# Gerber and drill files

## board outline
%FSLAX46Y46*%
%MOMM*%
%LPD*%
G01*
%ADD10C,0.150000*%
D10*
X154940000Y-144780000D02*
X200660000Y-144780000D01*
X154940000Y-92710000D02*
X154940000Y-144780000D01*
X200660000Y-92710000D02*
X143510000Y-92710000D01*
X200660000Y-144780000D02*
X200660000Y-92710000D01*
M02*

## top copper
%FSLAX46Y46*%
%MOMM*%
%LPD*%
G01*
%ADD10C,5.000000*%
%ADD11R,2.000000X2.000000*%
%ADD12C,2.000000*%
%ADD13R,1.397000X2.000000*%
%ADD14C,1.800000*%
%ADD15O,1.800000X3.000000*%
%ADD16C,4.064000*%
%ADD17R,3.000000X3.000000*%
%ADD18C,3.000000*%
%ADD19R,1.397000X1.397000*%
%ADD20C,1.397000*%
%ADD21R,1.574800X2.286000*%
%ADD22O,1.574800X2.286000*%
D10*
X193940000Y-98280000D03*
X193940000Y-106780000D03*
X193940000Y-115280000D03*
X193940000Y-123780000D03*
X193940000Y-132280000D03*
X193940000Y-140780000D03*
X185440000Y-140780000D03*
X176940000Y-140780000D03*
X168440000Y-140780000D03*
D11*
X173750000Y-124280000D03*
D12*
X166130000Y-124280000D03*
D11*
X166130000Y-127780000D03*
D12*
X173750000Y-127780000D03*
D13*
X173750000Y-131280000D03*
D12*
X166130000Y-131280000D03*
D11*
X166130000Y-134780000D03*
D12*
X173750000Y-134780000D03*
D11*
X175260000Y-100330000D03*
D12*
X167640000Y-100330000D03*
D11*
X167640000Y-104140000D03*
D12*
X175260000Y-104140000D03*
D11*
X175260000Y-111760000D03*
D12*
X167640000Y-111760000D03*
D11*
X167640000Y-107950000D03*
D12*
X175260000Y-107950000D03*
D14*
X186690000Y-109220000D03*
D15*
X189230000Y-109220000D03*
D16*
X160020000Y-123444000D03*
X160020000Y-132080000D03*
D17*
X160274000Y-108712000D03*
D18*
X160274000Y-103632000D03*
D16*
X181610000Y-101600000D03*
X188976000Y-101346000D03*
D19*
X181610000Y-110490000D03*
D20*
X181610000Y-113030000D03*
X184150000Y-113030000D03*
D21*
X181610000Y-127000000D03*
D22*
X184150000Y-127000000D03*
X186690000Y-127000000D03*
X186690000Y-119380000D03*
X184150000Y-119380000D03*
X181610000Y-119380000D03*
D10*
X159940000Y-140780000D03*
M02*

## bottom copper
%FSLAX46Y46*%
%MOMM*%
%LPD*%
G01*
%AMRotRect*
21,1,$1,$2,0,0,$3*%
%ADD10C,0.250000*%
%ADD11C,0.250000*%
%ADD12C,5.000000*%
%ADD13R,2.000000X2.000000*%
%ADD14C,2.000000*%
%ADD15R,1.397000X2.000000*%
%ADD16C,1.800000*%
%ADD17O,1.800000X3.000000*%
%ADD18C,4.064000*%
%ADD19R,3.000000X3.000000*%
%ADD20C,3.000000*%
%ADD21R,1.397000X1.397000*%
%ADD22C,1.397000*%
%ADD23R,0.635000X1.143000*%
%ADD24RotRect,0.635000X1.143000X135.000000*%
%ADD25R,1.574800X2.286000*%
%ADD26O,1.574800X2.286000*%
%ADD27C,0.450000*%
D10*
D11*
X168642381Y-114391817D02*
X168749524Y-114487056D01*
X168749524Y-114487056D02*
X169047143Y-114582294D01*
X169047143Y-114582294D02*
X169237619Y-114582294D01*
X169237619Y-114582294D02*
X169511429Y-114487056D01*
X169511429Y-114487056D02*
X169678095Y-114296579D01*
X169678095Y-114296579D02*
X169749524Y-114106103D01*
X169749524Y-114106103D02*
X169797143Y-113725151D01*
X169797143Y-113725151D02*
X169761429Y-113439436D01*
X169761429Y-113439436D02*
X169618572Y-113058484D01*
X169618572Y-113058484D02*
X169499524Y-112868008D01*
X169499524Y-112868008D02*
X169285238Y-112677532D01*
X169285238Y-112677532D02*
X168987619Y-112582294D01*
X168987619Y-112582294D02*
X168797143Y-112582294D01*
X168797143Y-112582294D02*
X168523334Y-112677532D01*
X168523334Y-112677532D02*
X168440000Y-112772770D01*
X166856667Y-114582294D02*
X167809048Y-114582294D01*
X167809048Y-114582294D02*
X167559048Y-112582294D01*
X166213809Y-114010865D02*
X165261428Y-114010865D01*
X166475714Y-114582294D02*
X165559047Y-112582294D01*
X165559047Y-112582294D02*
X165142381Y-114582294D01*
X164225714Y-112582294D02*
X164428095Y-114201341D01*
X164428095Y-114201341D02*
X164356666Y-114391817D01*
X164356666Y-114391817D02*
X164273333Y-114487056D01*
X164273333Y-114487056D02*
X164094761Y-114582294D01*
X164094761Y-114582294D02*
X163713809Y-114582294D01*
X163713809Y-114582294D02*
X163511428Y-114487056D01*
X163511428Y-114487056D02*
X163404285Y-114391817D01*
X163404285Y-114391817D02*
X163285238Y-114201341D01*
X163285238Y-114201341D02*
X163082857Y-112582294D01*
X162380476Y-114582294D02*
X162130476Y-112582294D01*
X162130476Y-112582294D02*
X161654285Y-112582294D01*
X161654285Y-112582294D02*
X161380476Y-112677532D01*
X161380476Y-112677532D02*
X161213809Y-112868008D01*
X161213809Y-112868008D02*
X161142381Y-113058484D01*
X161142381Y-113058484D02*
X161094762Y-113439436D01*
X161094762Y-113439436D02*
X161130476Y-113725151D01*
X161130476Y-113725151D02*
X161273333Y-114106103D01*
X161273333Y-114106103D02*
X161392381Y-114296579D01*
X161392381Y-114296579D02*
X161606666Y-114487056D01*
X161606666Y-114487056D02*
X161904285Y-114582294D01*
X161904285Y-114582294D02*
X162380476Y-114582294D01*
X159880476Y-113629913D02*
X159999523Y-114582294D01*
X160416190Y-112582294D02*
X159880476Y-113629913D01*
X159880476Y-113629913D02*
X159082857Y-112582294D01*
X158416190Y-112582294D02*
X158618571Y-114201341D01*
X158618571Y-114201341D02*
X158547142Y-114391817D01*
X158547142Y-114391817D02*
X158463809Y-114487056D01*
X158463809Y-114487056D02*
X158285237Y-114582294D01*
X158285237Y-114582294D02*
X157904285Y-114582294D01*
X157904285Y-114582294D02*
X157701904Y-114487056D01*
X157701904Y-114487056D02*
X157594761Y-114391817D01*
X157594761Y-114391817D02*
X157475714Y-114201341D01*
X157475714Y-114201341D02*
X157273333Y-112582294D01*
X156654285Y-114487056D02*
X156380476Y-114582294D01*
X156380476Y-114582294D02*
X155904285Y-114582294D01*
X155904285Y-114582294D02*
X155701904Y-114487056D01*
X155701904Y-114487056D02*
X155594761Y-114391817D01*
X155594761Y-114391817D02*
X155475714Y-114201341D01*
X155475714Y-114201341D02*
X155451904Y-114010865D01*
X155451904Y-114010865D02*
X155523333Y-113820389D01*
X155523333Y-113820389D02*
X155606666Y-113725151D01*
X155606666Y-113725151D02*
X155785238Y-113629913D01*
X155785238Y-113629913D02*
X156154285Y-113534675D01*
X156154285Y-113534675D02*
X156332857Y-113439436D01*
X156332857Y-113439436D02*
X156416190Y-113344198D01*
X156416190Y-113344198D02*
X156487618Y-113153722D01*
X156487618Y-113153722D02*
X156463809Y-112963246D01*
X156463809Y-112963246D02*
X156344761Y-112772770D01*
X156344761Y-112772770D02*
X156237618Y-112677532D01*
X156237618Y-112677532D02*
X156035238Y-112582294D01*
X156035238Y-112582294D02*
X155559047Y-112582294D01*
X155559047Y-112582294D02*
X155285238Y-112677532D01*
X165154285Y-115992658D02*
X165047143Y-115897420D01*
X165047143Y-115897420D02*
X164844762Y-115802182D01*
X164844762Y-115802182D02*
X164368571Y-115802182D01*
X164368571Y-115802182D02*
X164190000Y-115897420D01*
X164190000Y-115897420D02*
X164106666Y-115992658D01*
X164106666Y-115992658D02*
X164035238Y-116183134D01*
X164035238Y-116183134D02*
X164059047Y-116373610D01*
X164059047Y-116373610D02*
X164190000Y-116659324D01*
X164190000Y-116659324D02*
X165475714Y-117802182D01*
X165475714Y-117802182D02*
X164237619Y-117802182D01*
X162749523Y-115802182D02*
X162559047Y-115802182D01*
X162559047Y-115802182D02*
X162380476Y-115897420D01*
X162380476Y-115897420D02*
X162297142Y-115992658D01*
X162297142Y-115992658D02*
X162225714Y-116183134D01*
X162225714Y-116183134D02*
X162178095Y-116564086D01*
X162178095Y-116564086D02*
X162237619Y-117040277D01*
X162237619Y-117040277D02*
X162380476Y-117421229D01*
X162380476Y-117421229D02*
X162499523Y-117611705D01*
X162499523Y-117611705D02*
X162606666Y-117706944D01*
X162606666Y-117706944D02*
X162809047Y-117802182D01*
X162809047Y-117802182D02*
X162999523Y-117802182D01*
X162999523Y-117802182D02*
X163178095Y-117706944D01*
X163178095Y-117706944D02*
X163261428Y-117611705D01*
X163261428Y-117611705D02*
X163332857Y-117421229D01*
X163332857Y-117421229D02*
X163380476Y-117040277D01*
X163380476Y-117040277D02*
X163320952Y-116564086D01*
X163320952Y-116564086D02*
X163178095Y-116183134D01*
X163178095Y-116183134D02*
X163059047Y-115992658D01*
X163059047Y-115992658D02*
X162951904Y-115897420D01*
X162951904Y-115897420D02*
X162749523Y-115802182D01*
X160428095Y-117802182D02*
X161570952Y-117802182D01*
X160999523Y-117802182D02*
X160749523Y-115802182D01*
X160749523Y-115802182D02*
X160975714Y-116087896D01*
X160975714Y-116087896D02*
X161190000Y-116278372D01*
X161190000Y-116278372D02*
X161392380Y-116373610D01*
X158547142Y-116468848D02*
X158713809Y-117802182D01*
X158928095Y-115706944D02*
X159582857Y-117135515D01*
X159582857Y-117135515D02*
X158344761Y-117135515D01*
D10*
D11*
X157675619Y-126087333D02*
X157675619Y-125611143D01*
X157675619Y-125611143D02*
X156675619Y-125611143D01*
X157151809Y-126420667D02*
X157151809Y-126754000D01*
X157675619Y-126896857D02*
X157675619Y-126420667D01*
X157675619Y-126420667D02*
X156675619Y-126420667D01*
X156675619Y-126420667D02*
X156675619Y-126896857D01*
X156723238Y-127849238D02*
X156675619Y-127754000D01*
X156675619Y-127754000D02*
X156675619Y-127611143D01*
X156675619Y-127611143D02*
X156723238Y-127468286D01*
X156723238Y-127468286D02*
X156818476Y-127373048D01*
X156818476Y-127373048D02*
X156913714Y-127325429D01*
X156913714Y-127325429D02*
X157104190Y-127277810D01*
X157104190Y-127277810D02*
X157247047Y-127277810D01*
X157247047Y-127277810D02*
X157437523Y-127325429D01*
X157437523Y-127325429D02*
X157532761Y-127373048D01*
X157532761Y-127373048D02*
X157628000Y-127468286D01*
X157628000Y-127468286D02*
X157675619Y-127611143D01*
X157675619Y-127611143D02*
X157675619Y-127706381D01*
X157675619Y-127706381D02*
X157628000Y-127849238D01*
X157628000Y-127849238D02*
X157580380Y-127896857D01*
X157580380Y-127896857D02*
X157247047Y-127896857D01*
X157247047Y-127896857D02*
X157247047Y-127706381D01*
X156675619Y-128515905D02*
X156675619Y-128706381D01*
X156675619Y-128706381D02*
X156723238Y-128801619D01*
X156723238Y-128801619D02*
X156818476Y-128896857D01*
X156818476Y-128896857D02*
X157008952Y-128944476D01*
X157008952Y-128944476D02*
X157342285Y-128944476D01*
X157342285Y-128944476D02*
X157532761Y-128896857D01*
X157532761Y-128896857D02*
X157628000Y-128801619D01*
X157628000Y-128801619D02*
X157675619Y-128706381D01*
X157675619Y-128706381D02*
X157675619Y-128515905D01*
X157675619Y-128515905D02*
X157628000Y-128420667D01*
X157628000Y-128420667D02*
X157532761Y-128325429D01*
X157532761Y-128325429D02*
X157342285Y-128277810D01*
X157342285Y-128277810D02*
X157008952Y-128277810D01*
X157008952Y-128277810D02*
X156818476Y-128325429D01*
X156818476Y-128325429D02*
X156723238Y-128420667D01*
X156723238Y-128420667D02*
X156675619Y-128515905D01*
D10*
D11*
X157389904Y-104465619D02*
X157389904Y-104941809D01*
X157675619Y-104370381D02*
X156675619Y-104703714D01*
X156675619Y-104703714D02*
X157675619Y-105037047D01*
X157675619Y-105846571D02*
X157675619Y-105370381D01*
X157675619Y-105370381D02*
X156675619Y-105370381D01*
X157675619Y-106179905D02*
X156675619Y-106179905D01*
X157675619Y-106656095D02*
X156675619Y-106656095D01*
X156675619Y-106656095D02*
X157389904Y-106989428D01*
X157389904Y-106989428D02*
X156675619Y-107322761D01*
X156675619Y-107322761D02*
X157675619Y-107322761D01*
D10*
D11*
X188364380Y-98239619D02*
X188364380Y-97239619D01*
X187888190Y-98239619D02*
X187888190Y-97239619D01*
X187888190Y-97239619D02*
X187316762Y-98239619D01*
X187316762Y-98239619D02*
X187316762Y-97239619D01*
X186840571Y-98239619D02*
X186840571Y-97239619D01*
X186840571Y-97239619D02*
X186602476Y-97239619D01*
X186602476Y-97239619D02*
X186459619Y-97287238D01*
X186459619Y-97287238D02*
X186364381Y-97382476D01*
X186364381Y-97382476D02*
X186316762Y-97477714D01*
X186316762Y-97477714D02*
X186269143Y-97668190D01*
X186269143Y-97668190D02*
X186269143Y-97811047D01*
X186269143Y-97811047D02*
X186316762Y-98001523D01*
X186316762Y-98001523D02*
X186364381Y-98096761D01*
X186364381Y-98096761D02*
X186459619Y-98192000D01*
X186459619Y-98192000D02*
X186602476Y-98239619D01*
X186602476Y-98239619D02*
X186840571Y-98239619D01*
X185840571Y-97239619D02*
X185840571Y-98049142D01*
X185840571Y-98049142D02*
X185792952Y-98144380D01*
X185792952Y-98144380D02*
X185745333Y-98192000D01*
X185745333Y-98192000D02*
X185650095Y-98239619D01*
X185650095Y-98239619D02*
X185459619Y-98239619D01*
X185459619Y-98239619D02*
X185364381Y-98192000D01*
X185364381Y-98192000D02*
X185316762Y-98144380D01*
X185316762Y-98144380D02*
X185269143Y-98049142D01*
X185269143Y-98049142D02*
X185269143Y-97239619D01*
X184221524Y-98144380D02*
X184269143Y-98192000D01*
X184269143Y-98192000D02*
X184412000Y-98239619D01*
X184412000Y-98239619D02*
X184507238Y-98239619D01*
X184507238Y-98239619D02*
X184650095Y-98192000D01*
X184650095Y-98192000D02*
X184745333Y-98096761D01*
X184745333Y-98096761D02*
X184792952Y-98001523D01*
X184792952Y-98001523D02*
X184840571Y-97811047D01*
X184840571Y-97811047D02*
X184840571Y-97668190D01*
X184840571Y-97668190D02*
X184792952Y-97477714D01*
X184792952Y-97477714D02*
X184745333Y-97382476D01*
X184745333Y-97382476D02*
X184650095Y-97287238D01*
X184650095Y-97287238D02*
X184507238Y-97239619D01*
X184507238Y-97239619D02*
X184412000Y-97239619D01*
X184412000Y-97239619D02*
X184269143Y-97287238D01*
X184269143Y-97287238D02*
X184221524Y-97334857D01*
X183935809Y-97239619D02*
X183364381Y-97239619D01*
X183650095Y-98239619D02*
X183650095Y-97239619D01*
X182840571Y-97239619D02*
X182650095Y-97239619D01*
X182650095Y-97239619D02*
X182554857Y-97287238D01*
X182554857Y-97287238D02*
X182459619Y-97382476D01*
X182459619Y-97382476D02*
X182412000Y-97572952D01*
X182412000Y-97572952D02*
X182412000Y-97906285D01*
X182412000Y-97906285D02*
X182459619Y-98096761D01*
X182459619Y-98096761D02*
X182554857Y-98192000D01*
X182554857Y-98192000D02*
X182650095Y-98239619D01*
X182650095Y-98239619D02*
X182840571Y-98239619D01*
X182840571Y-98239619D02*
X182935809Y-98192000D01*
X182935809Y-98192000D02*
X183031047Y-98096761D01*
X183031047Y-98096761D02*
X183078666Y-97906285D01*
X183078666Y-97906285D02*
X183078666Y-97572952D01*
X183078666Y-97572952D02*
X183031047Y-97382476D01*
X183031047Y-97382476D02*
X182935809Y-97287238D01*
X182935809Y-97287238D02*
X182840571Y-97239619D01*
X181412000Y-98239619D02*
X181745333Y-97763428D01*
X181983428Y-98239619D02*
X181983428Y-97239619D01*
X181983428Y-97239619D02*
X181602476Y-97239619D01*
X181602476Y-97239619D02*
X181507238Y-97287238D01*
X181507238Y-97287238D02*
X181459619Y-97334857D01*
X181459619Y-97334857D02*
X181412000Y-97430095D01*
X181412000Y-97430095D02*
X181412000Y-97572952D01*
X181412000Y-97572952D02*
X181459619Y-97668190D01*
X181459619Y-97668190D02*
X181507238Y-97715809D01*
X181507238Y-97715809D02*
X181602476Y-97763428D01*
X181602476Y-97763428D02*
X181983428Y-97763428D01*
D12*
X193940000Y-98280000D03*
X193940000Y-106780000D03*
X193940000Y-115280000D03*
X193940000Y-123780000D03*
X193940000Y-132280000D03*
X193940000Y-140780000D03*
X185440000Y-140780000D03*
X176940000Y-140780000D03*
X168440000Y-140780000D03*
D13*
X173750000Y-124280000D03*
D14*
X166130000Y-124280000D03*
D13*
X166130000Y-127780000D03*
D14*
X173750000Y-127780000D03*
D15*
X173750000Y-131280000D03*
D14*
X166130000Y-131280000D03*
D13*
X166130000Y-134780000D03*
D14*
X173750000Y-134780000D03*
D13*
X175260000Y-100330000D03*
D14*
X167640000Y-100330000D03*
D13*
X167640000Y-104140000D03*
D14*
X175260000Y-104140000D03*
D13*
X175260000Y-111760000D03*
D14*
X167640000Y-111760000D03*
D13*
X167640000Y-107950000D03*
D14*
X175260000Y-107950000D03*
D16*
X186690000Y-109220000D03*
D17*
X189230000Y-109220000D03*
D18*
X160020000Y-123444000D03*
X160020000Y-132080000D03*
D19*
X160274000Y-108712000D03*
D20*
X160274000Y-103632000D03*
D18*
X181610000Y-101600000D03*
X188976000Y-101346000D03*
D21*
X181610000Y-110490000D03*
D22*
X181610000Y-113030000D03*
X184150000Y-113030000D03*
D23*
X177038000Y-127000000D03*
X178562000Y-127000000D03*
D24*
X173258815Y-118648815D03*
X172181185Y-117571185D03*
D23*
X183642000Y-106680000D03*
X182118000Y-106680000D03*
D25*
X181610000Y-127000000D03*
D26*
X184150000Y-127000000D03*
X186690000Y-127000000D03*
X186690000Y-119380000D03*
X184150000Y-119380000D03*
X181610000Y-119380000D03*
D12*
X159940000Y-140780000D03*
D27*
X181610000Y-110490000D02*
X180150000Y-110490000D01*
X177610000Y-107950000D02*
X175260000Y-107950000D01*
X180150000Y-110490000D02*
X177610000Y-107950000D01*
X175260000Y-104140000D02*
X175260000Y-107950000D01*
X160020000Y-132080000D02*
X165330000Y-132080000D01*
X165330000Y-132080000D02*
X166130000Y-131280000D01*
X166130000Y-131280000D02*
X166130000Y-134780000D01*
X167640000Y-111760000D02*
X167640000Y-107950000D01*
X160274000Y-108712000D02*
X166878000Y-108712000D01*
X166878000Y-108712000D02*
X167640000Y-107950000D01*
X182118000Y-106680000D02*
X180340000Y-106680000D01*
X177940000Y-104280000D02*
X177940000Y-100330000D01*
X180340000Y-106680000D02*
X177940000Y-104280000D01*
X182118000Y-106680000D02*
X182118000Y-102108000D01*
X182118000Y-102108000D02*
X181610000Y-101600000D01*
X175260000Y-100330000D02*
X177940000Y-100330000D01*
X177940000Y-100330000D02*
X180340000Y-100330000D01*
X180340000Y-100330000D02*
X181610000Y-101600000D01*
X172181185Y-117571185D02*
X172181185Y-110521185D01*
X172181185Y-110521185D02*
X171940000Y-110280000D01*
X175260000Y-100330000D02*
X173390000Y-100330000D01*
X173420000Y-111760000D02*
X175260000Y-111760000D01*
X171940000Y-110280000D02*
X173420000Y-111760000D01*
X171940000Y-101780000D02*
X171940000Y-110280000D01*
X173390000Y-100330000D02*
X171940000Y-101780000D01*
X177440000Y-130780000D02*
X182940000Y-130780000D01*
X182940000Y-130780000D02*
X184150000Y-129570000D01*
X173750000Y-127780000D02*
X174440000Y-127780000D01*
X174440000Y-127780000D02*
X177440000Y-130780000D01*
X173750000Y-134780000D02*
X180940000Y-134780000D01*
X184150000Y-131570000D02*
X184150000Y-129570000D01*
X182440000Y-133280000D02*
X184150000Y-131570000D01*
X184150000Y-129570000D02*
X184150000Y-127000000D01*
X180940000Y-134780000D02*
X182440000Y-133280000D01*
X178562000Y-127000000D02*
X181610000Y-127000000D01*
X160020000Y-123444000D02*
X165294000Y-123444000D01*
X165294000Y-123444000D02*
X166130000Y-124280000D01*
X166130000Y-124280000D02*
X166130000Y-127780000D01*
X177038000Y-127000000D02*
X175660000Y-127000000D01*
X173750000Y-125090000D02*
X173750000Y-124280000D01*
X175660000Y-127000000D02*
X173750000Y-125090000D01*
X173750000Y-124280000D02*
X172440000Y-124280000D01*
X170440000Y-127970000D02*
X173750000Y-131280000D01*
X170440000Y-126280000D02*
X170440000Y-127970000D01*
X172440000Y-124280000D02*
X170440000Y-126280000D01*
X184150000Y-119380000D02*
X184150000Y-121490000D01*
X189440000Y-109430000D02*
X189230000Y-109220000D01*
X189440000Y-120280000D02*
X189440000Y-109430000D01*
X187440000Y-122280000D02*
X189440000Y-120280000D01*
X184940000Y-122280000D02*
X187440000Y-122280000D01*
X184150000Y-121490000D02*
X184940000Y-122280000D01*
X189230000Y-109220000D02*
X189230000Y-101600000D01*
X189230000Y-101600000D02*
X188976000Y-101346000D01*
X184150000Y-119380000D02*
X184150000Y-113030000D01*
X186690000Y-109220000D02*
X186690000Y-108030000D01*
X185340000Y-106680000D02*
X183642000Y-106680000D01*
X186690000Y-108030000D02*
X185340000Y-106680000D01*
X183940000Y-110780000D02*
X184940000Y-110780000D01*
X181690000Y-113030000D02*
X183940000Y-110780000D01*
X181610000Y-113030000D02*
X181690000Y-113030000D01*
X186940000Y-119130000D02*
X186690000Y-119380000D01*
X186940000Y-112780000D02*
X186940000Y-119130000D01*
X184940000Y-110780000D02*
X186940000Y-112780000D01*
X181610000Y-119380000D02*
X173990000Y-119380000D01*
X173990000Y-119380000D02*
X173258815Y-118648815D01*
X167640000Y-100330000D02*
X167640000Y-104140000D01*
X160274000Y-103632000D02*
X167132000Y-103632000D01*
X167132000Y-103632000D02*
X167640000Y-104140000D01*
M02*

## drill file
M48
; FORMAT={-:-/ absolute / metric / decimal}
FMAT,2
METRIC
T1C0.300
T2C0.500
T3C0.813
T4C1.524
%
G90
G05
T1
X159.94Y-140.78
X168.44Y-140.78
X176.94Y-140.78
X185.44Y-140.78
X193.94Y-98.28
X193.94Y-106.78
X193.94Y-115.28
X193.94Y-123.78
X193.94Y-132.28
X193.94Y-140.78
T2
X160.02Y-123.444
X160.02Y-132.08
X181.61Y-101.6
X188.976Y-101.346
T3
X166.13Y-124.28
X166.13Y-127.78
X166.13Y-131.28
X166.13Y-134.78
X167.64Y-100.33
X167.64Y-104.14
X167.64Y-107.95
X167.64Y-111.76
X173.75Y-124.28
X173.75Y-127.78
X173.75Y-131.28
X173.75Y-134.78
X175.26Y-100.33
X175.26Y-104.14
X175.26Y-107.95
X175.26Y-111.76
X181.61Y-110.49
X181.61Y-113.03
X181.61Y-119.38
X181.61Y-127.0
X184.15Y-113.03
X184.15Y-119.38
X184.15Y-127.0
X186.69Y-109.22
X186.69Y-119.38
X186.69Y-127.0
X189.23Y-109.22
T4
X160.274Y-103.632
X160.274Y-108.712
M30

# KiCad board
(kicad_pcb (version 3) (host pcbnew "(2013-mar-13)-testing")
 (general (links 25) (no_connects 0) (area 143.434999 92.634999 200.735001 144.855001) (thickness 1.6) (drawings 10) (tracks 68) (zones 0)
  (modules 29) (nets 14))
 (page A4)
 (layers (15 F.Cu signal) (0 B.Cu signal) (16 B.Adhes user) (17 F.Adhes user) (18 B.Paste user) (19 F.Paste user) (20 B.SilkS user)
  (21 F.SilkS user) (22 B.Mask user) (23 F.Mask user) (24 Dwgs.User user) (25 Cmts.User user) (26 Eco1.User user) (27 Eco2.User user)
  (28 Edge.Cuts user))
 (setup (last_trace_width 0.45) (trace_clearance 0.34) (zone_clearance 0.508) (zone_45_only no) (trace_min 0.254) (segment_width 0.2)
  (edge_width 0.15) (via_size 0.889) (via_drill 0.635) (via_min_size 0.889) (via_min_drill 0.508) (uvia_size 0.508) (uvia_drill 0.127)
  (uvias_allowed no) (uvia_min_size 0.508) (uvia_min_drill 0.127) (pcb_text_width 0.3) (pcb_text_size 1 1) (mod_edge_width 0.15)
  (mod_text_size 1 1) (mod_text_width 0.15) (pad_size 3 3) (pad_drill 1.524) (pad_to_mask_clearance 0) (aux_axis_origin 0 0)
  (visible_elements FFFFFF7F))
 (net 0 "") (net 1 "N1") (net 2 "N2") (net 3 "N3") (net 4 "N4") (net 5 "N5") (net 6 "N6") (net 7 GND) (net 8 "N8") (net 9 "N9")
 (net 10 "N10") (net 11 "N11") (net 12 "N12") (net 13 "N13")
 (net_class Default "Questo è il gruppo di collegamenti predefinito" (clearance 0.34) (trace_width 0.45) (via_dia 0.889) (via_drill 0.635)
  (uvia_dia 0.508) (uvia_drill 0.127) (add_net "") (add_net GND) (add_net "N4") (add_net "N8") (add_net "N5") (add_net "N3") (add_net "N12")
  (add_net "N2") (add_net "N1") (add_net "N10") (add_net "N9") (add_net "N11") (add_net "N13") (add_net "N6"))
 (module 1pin (layer F.Cu) (at 193.94 98.28)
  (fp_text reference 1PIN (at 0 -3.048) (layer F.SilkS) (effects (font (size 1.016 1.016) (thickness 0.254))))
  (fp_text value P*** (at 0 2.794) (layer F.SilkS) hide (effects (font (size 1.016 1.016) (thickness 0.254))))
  (pad 1 thru_hole circle (at 0 0) (size 5 5) (drill 0.3) (layers *.Cu *.Mask F.SilkS)))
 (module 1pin (layer F.Cu) (at 193.94 106.78)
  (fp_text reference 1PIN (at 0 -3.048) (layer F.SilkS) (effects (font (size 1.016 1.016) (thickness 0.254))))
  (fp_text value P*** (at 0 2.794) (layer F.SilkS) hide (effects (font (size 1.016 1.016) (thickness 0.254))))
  (pad 1 thru_hole circle (at 0 0) (size 5 5) (drill 0.3) (layers *.Cu *.Mask F.SilkS)))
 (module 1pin (layer F.Cu) (at 193.94 115.28)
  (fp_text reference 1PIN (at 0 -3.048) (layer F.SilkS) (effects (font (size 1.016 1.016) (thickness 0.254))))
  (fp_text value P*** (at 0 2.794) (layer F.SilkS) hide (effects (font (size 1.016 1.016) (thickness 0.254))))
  (pad 1 thru_hole circle (at 0 0) (size 5 5) (drill 0.3) (layers *.Cu *.Mask F.SilkS)))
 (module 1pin (layer F.Cu) (at 193.94 123.78)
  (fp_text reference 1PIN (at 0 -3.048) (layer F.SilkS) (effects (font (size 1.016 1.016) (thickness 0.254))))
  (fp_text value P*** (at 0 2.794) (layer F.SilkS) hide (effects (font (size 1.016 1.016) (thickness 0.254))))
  (pad 1 thru_hole circle (at 0 0) (size 5 5) (drill 0.3) (layers *.Cu *.Mask F.SilkS)))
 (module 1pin (layer F.Cu) (at 193.94 132.28)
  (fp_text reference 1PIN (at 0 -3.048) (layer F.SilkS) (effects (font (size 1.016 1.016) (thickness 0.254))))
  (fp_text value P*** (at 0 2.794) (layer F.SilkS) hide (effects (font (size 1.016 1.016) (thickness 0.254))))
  (pad 1 thru_hole circle (at 0 0) (size 5 5) (drill 0.3) (layers *.Cu *.Mask F.SilkS)))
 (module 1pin (layer F.Cu) (at 193.94 140.78)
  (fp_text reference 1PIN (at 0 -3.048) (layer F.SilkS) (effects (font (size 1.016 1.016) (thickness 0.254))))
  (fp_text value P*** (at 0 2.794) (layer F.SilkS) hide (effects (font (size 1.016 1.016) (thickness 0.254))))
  (pad 1 thru_hole circle (at 0 0) (size 5 5) (drill 0.3) (layers *.Cu *.Mask F.SilkS)))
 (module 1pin (layer F.Cu) (at 185.44 140.78)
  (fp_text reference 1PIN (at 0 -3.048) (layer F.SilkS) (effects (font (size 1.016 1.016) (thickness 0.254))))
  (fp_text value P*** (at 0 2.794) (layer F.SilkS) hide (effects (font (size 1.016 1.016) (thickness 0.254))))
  (pad 1 thru_hole circle (at 0 0) (size 5 5) (drill 0.3) (layers *.Cu *.Mask F.SilkS)))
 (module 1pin (layer F.Cu) (at 176.94 140.78)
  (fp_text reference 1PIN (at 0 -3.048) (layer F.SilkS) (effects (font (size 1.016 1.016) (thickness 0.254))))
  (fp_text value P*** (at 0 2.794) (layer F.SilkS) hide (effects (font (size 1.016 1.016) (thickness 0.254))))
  (pad 1 thru_hole circle (at 0 0) (size 5 5) (drill 0.3) (layers *.Cu *.Mask F.SilkS)))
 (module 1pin (layer F.Cu) (at 168.44 140.78)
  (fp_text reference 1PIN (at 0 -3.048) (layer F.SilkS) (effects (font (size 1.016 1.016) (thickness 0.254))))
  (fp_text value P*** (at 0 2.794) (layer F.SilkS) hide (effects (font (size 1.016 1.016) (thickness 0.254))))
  (pad 1 thru_hole circle (at 0 0) (size 5 5) (drill 0.3) (layers *.Cu *.Mask F.SilkS)))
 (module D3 (layer F.Cu) (at 169.94 124.28)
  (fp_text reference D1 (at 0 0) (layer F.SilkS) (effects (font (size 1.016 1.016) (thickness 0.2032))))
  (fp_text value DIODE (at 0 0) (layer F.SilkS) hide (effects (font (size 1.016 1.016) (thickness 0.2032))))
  (pad 2 thru_hole rect (at 3.81 0) (size 2 2) (drill 0.8128) (layers *.Cu *.Mask F.SilkS) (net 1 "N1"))
  (pad 1 thru_hole circle (at -3.81 0) (size 2 2) (drill 0.8128) (layers *.Cu *.Mask F.SilkS) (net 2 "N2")))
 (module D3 (layer F.Cu) (at 169.94 127.78 180)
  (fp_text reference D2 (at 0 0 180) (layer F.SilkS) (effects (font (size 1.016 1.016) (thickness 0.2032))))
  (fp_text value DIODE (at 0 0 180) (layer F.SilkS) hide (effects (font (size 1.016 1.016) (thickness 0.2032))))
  (pad 2 thru_hole rect (at 3.81 0 180) (size 2 2) (drill 0.8128) (layers *.Cu *.Mask F.SilkS) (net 2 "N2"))
  (pad 1 thru_hole circle (at -3.81 0 180) (size 2 2) (drill 0.8128) (layers *.Cu *.Mask F.SilkS) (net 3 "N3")))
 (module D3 (layer F.Cu) (at 169.94 131.28)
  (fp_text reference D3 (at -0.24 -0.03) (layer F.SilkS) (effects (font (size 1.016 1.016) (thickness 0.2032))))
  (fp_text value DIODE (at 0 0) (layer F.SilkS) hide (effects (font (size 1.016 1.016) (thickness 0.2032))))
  (pad 2 thru_hole rect (at 3.81 0) (size 1.397 2) (drill 0.8128) (layers *.Cu *.Mask F.SilkS) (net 1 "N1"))
  (pad 1 thru_hole circle (at -3.81 0) (size 2 2) (drill 0.8128) (layers *.Cu *.Mask F.SilkS) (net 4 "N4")))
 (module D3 (layer F.Cu) (at 169.94 134.78 180)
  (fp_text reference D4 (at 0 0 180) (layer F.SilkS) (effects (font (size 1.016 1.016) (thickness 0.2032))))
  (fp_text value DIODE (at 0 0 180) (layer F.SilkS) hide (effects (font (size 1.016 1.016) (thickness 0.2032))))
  (pad 2 thru_hole rect (at 3.81 0 180) (size 2 2) (drill 0.8128) (layers *.Cu *.Mask F.SilkS) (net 4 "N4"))
  (pad 1 thru_hole circle (at -3.81 0 180) (size 2 2) (drill 0.8128) (layers *.Cu *.Mask F.SilkS) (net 3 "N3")))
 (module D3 (layer F.Cu) (at 171.45 100.33)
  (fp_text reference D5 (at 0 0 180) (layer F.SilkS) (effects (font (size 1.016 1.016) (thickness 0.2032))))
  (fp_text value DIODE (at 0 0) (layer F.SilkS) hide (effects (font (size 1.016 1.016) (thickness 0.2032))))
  (pad 2 thru_hole rect (at 3.81 0) (size 2 2) (drill 0.8128) (layers *.Cu *.Mask F.SilkS) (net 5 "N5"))
  (pad 1 thru_hole circle (at -3.81 0) (size 2 2) (drill 0.8128) (layers *.Cu *.Mask F.SilkS) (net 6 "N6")))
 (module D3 (layer F.Cu) (at 171.45 104.14 180)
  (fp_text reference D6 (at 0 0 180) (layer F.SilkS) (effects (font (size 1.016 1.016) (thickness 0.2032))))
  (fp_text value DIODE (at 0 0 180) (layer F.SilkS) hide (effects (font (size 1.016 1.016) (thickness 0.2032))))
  (pad 2 thru_hole rect (at 3.81 0 180) (size 2 2) (drill 0.8128) (layers *.Cu *.Mask F.SilkS) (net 6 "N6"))
  (pad 1 thru_hole circle (at -3.81 0 180) (size 2 2) (drill 0.8128) (layers *.Cu *.Mask F.SilkS) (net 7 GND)))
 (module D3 (layer F.Cu) (at 171.45 111.76)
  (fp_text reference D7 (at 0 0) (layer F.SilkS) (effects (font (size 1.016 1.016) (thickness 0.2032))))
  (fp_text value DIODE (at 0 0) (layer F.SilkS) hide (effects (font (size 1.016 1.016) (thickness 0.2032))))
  (pad 2 thru_hole rect (at 3.81 0) (size 2 2) (drill 0.8128) (layers *.Cu *.Mask F.SilkS) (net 5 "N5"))
  (pad 1 thru_hole circle (at -3.81 0) (size 2 2) (drill 0.8128) (layers *.Cu *.Mask F.SilkS) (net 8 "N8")))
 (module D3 (layer F.Cu) (at 171.45 107.95 180)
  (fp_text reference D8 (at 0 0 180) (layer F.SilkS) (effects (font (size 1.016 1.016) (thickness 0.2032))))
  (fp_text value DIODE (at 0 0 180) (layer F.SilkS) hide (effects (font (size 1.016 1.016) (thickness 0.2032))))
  (pad 2 thru_hole rect (at 3.81 0 180) (size 2 2) (drill 0.8128) (layers *.Cu *.Mask F.SilkS) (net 8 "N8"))
  (pad 1 thru_hole circle (at -3.81 0 180) (size 2 2) (drill 0.8128) (layers *.Cu *.Mask F.SilkS) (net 7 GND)))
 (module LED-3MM (layer F.Cu) (at 187.96 109.22)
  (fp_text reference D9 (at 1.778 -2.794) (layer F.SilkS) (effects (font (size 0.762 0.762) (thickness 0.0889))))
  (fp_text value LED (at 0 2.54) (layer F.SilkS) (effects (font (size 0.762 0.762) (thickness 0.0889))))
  (pad 1 thru_hole circle (at -1.27 0) (size 1.8 1.8) (drill 0.8128) (layers *.Cu *.Mask F.SilkS) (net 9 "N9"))
  (pad 2 thru_hole oval (at 1.27 0) (size 1.8 3) (drill 0.8128) (layers *.Cu *.Mask F.SilkS) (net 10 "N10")))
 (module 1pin (layer F.Cu) (at 160.02 123.444)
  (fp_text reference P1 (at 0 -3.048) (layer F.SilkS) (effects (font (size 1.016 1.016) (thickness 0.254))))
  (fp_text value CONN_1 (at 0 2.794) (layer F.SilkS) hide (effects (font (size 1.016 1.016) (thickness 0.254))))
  (pad 1 thru_hole circle (at 0 0) (size 4.064 4.064) (drill 0.5) (layers *.Cu *.Mask F.SilkS) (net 2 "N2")))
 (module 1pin (layer F.Cu) (at 160.02 132.08)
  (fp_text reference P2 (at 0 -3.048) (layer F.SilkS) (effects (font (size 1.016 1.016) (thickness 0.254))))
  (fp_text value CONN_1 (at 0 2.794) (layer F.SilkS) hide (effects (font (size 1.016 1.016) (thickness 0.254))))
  (pad 1 thru_hole circle (at 0 0) (size 4.064 4.064) (drill 0.5) (layers *.Cu *.Mask F.SilkS) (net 4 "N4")))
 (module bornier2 (layer F.Cu) (at 160.274 106.172 90)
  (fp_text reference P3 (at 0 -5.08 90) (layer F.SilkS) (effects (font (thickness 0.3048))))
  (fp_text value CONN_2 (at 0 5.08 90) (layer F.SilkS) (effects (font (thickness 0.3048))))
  (pad 1 thru_hole rect (at -2.54 0 90) (size 3 3) (drill 1.524) (layers *.Cu *.Mask F.SilkS) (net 8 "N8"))
  (pad 2 thru_hole circle (at 2.54 0 90) (size 3 3) (drill 1.524) (layers *.Cu *.Mask F.SilkS) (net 6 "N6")))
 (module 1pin (layer F.Cu) (at 181.61 101.6)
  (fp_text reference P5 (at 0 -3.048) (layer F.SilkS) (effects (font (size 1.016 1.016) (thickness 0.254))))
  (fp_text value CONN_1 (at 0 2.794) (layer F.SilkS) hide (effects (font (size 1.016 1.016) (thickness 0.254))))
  (pad 1 thru_hole circle (at 0 0) (size 4.064 4.064) (drill 0.5) (layers *.Cu *.Mask F.SilkS) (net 5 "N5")))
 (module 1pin (layer F.Cu) (at 188.976 101.346)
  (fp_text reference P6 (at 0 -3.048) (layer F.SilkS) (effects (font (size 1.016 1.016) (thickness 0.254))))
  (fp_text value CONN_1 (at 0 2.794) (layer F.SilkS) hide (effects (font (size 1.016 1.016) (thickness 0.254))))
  (pad 1 thru_hole circle (at 0 0) (size 4.064 4.064) (drill 0.5) (layers *.Cu *.Mask F.SilkS) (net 10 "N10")))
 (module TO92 (layer F.Cu) (at 182.88 111.76 90)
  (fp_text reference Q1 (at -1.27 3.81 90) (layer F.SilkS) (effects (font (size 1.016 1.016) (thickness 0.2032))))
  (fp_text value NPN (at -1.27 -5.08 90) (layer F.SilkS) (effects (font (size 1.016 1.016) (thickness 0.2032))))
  (pad 1 thru_hole rect (at 1.27 -1.27 90) (size 1.397 1.397) (drill 0.8128) (layers *.Cu *.Mask F.SilkS) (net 7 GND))
  (pad 2 thru_hole circle (at -1.27 -1.27 90) (size 1.397 1.397) (drill 0.8128) (layers *.Cu *.Mask F.SilkS) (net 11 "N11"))
  (pad 3 thru_hole circle (at -1.27 1.27 90) (size 1.397 1.397) (drill 0.8128) (layers *.Cu *.Mask F.SilkS) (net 10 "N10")))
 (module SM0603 (layer B.Cu) (at 177.8 127)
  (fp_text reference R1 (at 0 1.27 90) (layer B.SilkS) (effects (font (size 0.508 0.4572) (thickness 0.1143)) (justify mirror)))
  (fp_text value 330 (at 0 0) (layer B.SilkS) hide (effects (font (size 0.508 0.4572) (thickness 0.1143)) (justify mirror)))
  (pad 1 smd rect (at -0.762 0) (size 0.635 1.143) (layers B.Cu B.Paste B.Mask) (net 1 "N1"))
  (pad 2 smd rect (at 0.762 0) (size 0.635 1.143) (layers B.Cu B.Paste B.Mask) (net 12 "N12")))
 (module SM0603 (layer B.Cu) (at 172.72 118.11 135)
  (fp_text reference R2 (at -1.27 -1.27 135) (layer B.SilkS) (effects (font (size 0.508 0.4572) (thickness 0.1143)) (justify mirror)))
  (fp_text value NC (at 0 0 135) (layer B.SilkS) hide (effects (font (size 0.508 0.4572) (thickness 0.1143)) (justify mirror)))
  (pad 1 smd rect (at -0.762 0 135) (size 0.635 1.143) (layers B.Cu B.Paste B.Mask) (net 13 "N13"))
  (pad 2 smd rect (at 0.762 0 135) (size 0.635 1.143) (layers B.Cu B.Paste B.Mask) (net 5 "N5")))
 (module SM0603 (layer B.Cu) (at 182.88 106.68 180)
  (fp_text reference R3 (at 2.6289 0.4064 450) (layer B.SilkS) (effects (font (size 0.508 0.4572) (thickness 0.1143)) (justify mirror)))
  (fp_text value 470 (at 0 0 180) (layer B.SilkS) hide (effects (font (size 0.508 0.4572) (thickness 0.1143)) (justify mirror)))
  (pad 1 smd rect (at -0.762 0 180) (size 0.635 1.143) (layers B.Cu B.Paste B.Mask) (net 9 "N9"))
  (pad 2 smd rect (at 0.762 0 180) (size 0.635 1.143) (layers B.Cu B.Paste B.Mask) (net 5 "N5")))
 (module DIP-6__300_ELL (layer F.Cu) (at 184.15 123.19)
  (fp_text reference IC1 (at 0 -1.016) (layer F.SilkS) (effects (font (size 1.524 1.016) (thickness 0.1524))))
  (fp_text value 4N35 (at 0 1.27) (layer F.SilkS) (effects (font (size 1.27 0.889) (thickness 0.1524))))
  (pad 1 thru_hole rect (at -2.54 3.81) (size 1.5748 2.286) (drill 0.8128) (layers *.Cu *.Mask F.SilkS) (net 12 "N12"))
  (pad 2 thru_hole oval (at 0 3.81) (size 1.5748 2.286) (drill 0.8128) (layers *.Cu *.Mask F.SilkS) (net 3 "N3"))
  (pad 3 thru_hole oval (at 2.54 3.81) (size 1.5748 2.286) (drill 0.8128) (layers *.Cu *.Mask F.SilkS))
  (pad 4 thru_hole oval (at 2.54 -3.81) (size 1.5748 2.286) (drill 0.8128) (layers *.Cu *.Mask F.SilkS) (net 11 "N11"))
  (pad 5 thru_hole oval (at 0 -3.81) (size 1.5748 2.286) (drill 0.8128) (layers *.Cu *.Mask F.SilkS) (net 10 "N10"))
  (pad 6 thru_hole oval (at -2.54 -3.81) (size 1.5748 2.286) (drill 0.8128) (layers *.Cu *.Mask F.SilkS) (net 13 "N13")))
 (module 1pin (layer F.Cu) (at 159.94 140.78)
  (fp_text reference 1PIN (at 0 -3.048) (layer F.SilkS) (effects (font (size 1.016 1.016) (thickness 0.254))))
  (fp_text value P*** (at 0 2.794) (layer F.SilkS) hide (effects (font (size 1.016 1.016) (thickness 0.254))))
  (pad 1 thru_hole circle (at 0 0) (size 5 5) (drill 0.3) (layers *.Cu *.Mask F.SilkS)))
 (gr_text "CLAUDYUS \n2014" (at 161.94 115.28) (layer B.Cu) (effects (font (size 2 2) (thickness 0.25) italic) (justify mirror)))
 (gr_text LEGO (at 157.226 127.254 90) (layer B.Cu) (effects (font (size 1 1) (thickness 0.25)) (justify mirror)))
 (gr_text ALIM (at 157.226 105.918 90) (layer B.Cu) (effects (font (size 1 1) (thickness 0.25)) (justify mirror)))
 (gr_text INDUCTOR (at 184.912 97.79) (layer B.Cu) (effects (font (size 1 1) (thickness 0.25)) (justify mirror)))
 (gr_line (start 154.94 144.78) (end 200.66 144.78) (angle 90) (layer Edge.Cuts) (width 0.15))
 (gr_line (start 154.94 92.71) (end 154.94 144.78) (angle 90) (layer Edge.Cuts) (width 0.15))
 (gr_line (start 200.66 92.71) (end 143.51 92.71) (angle 90) (layer Edge.Cuts) (width 0.15))
 (gr_line (start 200.66 144.78) (end 200.66 92.71) (angle 90) (layer Edge.Cuts) (width 0.15))
 (segment (start 181.61 110.49) (end 180.15 110.49) (width 0.45) (layer B.Cu) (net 7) (status 400000))
 (segment (start 177.61 107.95) (end 175.26 107.95) (width 0.45) (layer B.Cu) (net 7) (status 800000))
 (segment (start 180.15 110.49) (end 177.61 107.95) (width 0.45) (layer B.Cu) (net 7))
 (segment (start 175.26 104.14) (end 175.26 107.95) (width 0.45) (layer B.Cu) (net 7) (status C00000))
 (segment (start 160.02 132.08) (end 165.33 132.08) (width 0.45) (layer B.Cu) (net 4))
 (segment (start 165.33 132.08) (end 166.13 131.28) (width 0.45) (layer B.Cu) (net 4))
 (segment (start 166.13 131.28) (end 166.13 134.78) (width 0.45) (layer B.Cu) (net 4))
 (segment (start 167.64 111.76) (end 167.64 107.95) (width 0.45) (layer B.Cu) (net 8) (status C00000))
 (segment (start 160.274 108.712) (end 166.878 108.712) (width 0.45) (layer B.Cu) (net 8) (status 400000))
 (segment (start 166.878 108.712) (end 167.64 107.95) (width 0.45) (layer B.Cu) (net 8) (status 800000))
 (segment (start 182.118 106.68) (end 180.34 106.68) (width 0.45) (layer B.Cu) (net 5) (status 400000))
 (segment (start 177.94 104.28) (end 177.94 100.33) (width 0.45) (layer B.Cu) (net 5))
 (segment (start 180.34 106.68) (end 177.94 104.28) (width 0.45) (layer B.Cu) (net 5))
 (segment (start 182.118 106.68) (end 182.118 102.108) (width 0.45) (layer B.Cu) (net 5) (status C00000))
 (segment (start 182.118 102.108) (end 181.61 101.6) (width 0.45) (layer B.Cu) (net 5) (status C00000))
 (segment (start 175.26 100.33) (end 177.94 100.33) (width 0.45) (layer B.Cu) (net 5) (status 400000))
 (segment (start 177.94 100.33) (end 180.34 100.33) (width 0.45) (layer B.Cu) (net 5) (status 800000))
 (segment (start 180.34 100.33) (end 181.61 101.6) (width 0.45) (layer B.Cu) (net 5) (status C00000))
 (segment (start 172.181185 117.571185) (end 172.181185 110.521185) (width 0.45) (layer B.Cu) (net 5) (status 400000))
 (segment (start 172.181185 110.521185) (end 171.94 110.28) (width 0.45) (layer B.Cu) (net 5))
 (segment (start 175.26 100.33) (end 173.39 100.33) (width 0.45) (layer B.Cu) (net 5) (status 400000))
 (segment (start 173.42 111.76) (end 175.26 111.76) (width 0.45) (layer B.Cu) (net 5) (status 800000))
 (segment (start 171.94 110.28) (end 173.42 111.76) (width 0.45) (layer B.Cu) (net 5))
 (segment (start 171.94 101.78) (end 171.94 110.28) (width 0.45) (layer B.Cu) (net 5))
 (segment (start 173.39 100.33) (end 171.94 101.78) (width 0.45) (layer B.Cu) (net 5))
 (segment (start 177.44 130.78) (end 182.94 130.78) (width 0.45) (layer B.Cu) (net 3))
 (segment (start 182.94 130.78) (end 184.15 129.57) (width 0.45) (layer B.Cu) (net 3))
 (segment (start 173.75 127.78) (end 174.44 127.78) (width 0.45) (layer B.Cu) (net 3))
 (segment (start 174.44 127.78) (end 177.44 130.78) (width 0.45) (layer B.Cu) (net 3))
 (segment (start 173.75 134.78) (end 180.94 134.78) (width 0.45) (layer B.Cu) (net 3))
 (segment (start 184.15 131.57) (end 184.15 129.57) (width 0.45) (layer B.Cu) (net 3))
 (segment (start 182.44 133.28) (end 184.15 131.57) (width 0.45) (layer B.Cu) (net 3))
 (segment (start 184.15 129.57) (end 184.15 127) (width 0.45) (layer B.Cu) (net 3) (status 2))
 (segment (start 180.94 134.78) (end 182.44 133.28) (width 0.45) (layer B.Cu) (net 3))
 (segment (start 178.562 127) (end 181.61 127) (width 0.45) (layer B.Cu) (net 12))
 (segment (start 160.02 123.444) (end 165.294 123.444) (width 0.45) (layer B.Cu) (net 2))
 (segment (start 165.294 123.444) (end 166.13 124.28) (width 0.45) (layer B.Cu) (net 2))
 (segment (start 166.13 124.28) (end 166.13 127.78) (width 0.45) (layer B.Cu) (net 2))
 (segment (start 177.038 127) (end 175.66 127) (width 0.45) (layer B.Cu) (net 1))
 (segment (start 173.75 125.09) (end 173.75 124.28) (width 0.45) (layer B.Cu) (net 1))
 (segment (start 175.66 127) (end 173.75 125.09) (width 0.45) (layer B.Cu) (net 1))
 (segment (start 173.75 124.28) (end 172.44 124.28) (width 0.45) (layer B.Cu) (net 1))
 (segment (start 170.44 127.97) (end 173.75 131.28) (width 0.45) (layer B.Cu) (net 1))
 (segment (start 170.44 126.28) (end 170.44 127.97) (width 0.45) (layer B.Cu) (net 1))
 (segment (start 172.44 124.28) (end 170.44 126.28) (width 0.45) (layer B.Cu) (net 1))
 (segment (start 184.15 119.38) (end 184.15 121.49) (width 0.45) (layer B.Cu) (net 10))
 (segment (start 189.44 109.43) (end 189.23 109.22) (width 0.45) (layer B.Cu) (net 10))
 (segment (start 189.44 120.28) (end 189.44 109.43) (width 0.45) (layer B.Cu) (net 10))
 (segment (start 187.44 122.28) (end 189.44 120.28) (width 0.45) (layer B.Cu) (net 10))
 (segment (start 184.94 122.28) (end 187.44 122.28) (width 0.45) (layer B.Cu) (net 10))
 (segment (start 184.15 121.49) (end 184.94 122.28) (width 0.45) (layer B.Cu) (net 10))
 (segment (start 189.23 109.22) (end 189.23 101.6) (width 0.45) (layer B.Cu) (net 10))
 (segment (start 189.23 101.6) (end 188.976 101.346) (width 0.45) (layer B.Cu) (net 10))
 (segment (start 184.15 119.38) (end 184.15 113.03) (width 0.45) (layer B.Cu) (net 10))
 (segment (start 186.69 109.22) (end 186.69 108.03) (width 0.45) (layer B.Cu) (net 9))
 (segment (start 185.34 106.68) (end 183.642 106.68) (width 0.45) (layer B.Cu) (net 9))
 (segment (start 186.69 108.03) (end 185.34 106.68) (width 0.45) (layer B.Cu) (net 9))
 (segment (start 183.94 110.78) (end 184.94 110.78) (width 0.45) (layer B.Cu) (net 11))
 (segment (start 181.69 113.03) (end 183.94 110.78) (width 0.45) (layer B.Cu) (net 11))
 (segment (start 181.61 113.03) (end 181.69 113.03) (width 0.45) (layer B.Cu) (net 11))
 (segment (start 186.94 119.13) (end 186.69 119.38) (width 0.45) (layer B.Cu) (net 11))
 (segment (start 186.94 112.78) (end 186.94 119.13) (width 0.45) (layer B.Cu) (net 11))
 (segment (start 184.94 110.78) (end 186.94 112.78) (width 0.45) (layer B.Cu) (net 11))
 (segment (start 181.61 119.38) (end 173.99 119.38) (width 0.45) (layer B.Cu) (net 13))
 (segment (start 173.99 119.38) (end 173.258815 118.648815) (width 0.45) (layer B.Cu) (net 13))
 (segment (start 167.64 100.33) (end 167.64 104.14) (width 0.45) (layer B.Cu) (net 6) (status C00000))
 (segment (start 160.274 103.632) (end 167.132 103.632) (width 0.45) (layer B.Cu) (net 6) (status C00000))
 (segment (start 167.132 103.632) (end 167.64 104.14) (width 0.45) (layer B.Cu) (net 6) (status C00000)))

